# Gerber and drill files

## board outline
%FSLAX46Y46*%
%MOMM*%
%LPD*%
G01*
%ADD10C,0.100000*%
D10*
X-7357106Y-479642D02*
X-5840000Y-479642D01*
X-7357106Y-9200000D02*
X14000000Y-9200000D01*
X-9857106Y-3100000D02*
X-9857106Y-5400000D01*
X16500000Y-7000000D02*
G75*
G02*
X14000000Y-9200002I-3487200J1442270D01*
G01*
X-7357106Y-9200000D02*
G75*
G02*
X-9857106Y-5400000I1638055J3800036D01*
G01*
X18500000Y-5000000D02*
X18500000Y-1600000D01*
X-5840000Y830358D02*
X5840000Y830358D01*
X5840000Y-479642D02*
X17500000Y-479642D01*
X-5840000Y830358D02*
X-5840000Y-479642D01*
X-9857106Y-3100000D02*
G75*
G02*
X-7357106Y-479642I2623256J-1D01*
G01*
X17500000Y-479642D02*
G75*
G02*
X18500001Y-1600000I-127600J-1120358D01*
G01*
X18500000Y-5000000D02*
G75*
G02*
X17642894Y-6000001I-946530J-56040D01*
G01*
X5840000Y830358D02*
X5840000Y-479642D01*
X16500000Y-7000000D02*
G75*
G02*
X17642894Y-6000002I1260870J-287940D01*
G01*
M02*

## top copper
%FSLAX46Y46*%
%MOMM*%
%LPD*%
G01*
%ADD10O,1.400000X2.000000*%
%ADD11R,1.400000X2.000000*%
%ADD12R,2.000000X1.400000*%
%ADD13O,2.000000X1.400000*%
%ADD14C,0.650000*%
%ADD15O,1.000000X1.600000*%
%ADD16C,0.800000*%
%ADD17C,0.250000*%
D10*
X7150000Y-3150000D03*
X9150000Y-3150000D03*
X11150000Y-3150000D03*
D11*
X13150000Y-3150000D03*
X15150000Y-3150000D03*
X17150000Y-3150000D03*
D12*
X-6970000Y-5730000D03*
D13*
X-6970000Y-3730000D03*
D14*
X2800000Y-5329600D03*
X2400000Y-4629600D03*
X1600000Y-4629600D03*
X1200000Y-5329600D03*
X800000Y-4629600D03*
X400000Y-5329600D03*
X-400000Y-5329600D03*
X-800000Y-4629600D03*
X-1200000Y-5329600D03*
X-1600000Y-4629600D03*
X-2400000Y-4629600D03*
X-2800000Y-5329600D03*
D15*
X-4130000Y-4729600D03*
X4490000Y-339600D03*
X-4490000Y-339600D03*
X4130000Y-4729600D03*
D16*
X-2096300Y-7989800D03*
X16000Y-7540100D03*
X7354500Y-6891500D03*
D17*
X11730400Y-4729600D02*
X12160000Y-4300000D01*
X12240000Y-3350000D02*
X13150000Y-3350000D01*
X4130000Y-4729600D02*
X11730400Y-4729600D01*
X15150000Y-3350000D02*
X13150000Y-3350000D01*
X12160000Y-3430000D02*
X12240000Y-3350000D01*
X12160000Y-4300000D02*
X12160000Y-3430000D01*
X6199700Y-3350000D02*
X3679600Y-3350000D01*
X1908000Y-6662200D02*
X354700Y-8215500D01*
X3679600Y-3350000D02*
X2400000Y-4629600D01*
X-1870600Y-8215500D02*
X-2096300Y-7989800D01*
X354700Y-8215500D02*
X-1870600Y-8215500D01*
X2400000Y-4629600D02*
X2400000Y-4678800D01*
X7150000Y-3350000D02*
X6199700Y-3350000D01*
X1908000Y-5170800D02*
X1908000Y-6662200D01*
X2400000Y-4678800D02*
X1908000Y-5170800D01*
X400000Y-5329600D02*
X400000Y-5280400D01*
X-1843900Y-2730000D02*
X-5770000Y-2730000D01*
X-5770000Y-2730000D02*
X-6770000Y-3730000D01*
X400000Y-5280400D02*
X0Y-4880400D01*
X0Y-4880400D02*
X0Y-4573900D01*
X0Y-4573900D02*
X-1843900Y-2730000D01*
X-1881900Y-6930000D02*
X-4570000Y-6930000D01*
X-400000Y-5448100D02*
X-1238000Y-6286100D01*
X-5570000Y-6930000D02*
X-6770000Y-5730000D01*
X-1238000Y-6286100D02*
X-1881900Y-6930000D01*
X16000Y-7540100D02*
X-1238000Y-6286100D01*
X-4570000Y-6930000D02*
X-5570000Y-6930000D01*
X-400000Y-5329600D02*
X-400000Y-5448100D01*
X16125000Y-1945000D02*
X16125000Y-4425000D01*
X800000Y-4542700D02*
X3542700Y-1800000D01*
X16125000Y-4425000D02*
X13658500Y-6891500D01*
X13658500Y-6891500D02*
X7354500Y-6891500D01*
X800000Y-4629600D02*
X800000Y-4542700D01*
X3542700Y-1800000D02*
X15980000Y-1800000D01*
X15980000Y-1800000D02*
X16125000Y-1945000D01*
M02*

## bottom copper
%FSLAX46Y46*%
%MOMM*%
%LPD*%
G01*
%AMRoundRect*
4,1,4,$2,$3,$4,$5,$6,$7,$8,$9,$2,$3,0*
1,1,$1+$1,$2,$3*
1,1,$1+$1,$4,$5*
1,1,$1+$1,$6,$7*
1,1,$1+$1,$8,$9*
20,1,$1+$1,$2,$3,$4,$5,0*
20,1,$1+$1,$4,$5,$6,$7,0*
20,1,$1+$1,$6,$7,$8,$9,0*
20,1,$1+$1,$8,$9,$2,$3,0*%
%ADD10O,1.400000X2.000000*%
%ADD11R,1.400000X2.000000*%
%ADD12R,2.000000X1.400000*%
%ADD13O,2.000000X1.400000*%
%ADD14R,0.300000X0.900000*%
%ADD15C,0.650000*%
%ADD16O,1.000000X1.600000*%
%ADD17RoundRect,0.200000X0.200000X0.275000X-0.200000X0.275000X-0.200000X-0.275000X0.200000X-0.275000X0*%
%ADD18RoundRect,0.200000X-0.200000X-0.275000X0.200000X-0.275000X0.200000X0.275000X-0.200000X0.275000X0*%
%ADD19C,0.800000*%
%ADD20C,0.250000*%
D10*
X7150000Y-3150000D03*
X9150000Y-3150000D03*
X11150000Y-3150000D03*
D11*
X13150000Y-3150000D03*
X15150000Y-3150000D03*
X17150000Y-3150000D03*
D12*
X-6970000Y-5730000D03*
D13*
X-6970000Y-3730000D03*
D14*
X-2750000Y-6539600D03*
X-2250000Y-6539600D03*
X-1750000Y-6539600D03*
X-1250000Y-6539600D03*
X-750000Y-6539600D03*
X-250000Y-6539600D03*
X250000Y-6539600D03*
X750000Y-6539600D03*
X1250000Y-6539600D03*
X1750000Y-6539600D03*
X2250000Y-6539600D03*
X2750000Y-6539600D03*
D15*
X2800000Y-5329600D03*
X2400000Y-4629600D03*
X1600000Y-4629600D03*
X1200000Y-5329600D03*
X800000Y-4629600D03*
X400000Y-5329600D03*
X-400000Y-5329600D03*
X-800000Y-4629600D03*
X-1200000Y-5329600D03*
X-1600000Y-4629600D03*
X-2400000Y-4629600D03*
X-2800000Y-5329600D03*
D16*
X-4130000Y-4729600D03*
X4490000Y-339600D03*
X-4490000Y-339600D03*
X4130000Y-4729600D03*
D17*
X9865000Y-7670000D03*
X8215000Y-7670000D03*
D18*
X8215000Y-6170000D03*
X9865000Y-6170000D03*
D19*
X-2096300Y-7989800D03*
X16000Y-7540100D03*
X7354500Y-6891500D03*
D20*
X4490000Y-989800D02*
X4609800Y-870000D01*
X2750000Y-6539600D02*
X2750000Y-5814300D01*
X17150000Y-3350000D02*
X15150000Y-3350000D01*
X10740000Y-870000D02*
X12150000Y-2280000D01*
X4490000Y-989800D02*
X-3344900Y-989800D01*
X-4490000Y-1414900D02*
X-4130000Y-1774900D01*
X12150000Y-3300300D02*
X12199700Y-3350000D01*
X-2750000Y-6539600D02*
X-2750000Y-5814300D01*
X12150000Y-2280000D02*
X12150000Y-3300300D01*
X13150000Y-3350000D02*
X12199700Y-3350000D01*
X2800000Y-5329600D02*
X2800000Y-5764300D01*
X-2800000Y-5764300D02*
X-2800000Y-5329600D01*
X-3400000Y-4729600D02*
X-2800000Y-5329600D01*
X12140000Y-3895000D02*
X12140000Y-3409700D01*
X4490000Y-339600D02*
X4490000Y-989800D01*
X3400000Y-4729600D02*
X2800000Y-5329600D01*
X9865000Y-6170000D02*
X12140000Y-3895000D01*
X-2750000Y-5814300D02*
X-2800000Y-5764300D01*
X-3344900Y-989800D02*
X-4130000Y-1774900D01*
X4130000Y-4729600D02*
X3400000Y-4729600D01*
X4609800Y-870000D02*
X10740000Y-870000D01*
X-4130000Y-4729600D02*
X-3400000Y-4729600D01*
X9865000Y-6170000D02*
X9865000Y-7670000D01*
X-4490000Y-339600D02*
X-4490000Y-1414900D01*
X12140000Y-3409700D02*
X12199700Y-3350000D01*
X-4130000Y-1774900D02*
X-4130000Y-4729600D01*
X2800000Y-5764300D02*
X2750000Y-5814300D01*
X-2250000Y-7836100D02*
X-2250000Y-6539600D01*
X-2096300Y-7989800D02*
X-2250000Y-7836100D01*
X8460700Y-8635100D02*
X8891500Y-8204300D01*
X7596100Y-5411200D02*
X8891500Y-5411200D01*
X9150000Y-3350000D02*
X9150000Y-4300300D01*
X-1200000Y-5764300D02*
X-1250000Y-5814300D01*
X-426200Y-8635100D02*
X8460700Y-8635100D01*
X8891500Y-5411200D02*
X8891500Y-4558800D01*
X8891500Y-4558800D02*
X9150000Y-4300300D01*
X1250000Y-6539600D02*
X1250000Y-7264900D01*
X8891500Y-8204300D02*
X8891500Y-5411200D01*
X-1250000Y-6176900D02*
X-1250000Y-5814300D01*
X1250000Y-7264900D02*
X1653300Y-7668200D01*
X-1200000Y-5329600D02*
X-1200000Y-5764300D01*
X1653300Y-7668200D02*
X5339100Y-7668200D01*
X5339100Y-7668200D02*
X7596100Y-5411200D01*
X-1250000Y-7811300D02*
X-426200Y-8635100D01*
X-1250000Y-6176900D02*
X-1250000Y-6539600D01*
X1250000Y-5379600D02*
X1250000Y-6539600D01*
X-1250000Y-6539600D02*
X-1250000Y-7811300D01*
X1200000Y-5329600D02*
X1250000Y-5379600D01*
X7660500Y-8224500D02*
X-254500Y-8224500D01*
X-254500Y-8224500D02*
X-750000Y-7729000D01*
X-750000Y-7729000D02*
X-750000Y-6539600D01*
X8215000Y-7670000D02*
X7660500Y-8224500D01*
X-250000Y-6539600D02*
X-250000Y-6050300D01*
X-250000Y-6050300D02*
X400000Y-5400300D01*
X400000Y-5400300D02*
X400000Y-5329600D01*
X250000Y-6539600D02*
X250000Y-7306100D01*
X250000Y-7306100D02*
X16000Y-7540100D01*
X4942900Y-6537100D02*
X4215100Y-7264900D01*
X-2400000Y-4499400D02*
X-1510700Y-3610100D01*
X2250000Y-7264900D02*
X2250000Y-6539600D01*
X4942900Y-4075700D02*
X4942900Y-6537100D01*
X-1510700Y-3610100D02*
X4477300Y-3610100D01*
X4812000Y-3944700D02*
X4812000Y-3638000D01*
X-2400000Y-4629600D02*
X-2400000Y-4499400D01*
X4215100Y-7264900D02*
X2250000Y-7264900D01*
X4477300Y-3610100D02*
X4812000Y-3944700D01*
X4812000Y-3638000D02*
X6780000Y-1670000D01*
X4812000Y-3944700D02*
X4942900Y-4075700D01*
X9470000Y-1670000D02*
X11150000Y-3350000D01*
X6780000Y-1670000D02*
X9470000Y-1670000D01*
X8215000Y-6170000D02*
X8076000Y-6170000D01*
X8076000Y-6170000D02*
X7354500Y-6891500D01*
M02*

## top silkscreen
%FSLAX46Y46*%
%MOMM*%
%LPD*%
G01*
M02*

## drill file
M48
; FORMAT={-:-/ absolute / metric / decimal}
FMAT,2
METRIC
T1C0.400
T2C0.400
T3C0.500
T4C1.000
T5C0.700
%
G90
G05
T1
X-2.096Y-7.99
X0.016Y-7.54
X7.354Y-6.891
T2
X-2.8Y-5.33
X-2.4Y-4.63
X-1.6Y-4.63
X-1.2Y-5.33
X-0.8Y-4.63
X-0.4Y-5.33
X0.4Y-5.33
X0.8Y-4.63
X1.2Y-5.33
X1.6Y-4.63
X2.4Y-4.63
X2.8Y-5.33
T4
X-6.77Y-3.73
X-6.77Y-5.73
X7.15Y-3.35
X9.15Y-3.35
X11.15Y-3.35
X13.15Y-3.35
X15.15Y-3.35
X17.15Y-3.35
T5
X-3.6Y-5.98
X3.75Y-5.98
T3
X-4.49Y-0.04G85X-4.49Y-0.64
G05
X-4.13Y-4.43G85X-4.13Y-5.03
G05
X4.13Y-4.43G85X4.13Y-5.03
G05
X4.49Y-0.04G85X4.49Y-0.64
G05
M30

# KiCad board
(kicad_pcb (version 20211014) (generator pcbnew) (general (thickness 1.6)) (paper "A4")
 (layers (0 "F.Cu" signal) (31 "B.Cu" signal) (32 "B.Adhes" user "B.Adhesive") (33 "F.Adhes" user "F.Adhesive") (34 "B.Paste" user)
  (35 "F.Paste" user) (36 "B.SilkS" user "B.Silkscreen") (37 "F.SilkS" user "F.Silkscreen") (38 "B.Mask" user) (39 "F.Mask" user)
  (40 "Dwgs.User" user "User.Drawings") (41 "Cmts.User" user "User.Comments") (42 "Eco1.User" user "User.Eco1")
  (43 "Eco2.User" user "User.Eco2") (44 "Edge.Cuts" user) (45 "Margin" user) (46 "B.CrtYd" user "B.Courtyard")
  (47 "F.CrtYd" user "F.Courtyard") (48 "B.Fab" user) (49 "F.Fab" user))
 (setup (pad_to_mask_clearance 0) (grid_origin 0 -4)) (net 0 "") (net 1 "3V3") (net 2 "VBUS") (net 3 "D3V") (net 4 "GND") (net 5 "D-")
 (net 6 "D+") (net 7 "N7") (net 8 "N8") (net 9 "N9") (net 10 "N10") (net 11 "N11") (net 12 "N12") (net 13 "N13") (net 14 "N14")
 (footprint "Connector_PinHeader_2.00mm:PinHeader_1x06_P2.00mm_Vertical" (layer "F.Cu") (at 7.15 3.35 90)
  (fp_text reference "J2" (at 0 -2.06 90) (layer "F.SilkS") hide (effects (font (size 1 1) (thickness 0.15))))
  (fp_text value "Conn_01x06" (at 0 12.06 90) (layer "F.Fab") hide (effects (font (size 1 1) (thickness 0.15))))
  (pad "1" thru_hole oval locked (at 0 0 90) (size 2 1.4) (drill 1 (offset 0.2 0)) (layers *.Cu *.Mask) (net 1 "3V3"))
  (pad "2" thru_hole oval locked (at 0 2 90) (size 2 1.4) (drill 1 (offset 0.2 0)) (layers *.Cu *.Mask) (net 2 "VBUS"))
  (pad "3" thru_hole oval locked (at 0 4 90) (size 2 1.4) (drill 1 (offset 0.2 0)) (layers *.Cu *.Mask) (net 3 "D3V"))
  (pad "4" thru_hole rect locked (at 0 6 90) (size 2 1.4) (drill 1 (offset 0.2 0)) (layers *.Cu *.Mask) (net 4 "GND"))
  (pad "5" thru_hole rect locked (at 0 8 90) (size 2 1.4) (drill 1 (offset 0.2 0)) (layers *.Cu *.Mask) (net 4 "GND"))
  (pad "6" thru_hole rect locked (at 0 10 90) (size 2 1.4) (drill 1 (offset 0.2 0)) (layers *.Cu *.Mask) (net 4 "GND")))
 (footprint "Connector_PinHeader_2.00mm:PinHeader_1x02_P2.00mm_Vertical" (layer "F.Cu") (at -6.77 5.73 180)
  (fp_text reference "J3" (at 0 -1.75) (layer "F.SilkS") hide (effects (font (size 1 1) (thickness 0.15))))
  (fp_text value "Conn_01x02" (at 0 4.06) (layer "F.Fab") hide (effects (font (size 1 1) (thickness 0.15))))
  (pad "1" thru_hole rect locked (at 0 0 180) (size 2 1.4) (drill 1 (offset 0.2 0)) (layers *.Cu *.Mask) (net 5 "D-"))
  (pad "2" thru_hole oval locked (at 0 2 180) (size 2 1.4) (drill 1 (offset 0.2 0)) (layers *.Cu *.Mask) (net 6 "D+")))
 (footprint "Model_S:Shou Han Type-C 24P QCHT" (layer "B.Cu") (at 0 -1.5204)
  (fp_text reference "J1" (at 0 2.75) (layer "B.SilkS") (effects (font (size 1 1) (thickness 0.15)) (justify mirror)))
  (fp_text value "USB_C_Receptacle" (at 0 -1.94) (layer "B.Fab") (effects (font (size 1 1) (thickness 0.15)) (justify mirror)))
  (pad "" np_thru_hole circle (at -3.6 7.5) (size 0.7 0.7) (drill 0.7) (layers *.Cu *.Mask))
  (pad "" np_thru_hole circle (at 3.75 7.5) (size 0.7 0.7) (drill 0.7) (layers *.Cu *.Mask))
  (pad "A1" smd rect (at -2.75 8.06) (size 0.3 0.9) (layers "B.Cu" "B.Paste" "B.Mask") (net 4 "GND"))
  (pad "A2" smd rect (at -2.25 8.06) (size 0.3 0.9) (layers "B.Cu" "B.Paste" "B.Mask") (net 1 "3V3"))
  (pad "A3" smd rect (at -1.75 8.06) (size 0.3 0.9) (layers "B.Cu" "B.Paste" "B.Mask") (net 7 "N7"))
  (pad "A4" smd rect (at -1.25 8.06) (size 0.3 0.9) (layers "B.Cu" "B.Paste" "B.Mask") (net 2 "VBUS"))
  (pad "A5" smd rect (at -0.75 8.06) (size 0.3 0.9) (layers "B.Cu" "B.Paste" "B.Mask") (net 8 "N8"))
  (pad "A6" smd rect (at -0.25 8.06) (size 0.3 0.9) (layers "B.Cu" "B.Paste" "B.Mask") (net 6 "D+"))
  (pad "A7" smd rect (at 0.25 8.06) (size 0.3 0.9) (layers "B.Cu" "B.Paste" "B.Mask") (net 5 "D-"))
  (pad "A8" smd rect (at 0.75 8.06) (size 0.3 0.9) (layers "B.Cu" "B.Paste" "B.Mask") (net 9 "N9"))
  (pad "A9" smd rect (at 1.25 8.06) (size 0.3 0.9) (layers "B.Cu" "B.Paste" "B.Mask") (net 2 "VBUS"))
  (pad "A10" smd rect (at 1.75 8.06) (size 0.3 0.9) (layers "B.Cu" "B.Paste" "B.Mask") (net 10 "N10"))
  (pad "A11" smd rect (at 2.25 8.06) (size 0.3 0.9) (layers "B.Cu" "B.Paste" "B.Mask") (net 3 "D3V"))
  (pad "A12" smd rect (at 2.75 8.06) (size 0.3 0.9) (layers "B.Cu" "B.Paste" "B.Mask") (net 4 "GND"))
  (pad "B1" thru_hole circle (at 2.8 6.85) (size 0.65 0.65) (drill 0.4) (layers *.Cu *.Mask) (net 4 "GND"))
  (pad "B2" thru_hole circle (at 2.4 6.15) (size 0.65 0.65) (drill 0.4) (layers *.Cu *.Mask) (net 1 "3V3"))
  (pad "B3" thru_hole circle (at 1.6 6.15) (size 0.65 0.65) (drill 0.4) (layers *.Cu *.Mask) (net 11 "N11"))
  (pad "B4" thru_hole circle (at 1.2 6.85) (size 0.65 0.65) (drill 0.4) (layers *.Cu *.Mask) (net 2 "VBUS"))
  (pad "B5" thru_hole circle (at 0.8 6.15) (size 0.65 0.65) (drill 0.4) (layers *.Cu *.Mask) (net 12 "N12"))
  (pad "B6" thru_hole circle (at 0.4 6.85) (size 0.65 0.65) (drill 0.4) (layers *.Cu *.Mask) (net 6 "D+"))
  (pad "B7" thru_hole circle (at -0.4 6.85) (size 0.65 0.65) (drill 0.4) (layers *.Cu *.Mask) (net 5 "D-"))
  (pad "B8" thru_hole circle (at -0.8 6.15) (size 0.65 0.65) (drill 0.4) (layers *.Cu *.Mask) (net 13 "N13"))
  (pad "B9" thru_hole circle (at -1.2 6.85) (size 0.65 0.65) (drill 0.4) (layers *.Cu *.Mask) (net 2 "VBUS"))
  (pad "B10" thru_hole circle (at -1.6 6.15) (size 0.65 0.65) (drill 0.4) (layers *.Cu *.Mask) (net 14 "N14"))
  (pad "B11" thru_hole circle (at -2.4 6.15) (size 0.65 0.65) (drill 0.4) (layers *.Cu *.Mask) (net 3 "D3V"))
  (pad "B12" thru_hole circle (at -2.8 6.85) (size 0.65 0.65) (drill 0.4) (layers *.Cu *.Mask) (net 4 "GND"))
  (pad "S1" thru_hole oval (at -4.13 6.25) (size 1 1.6) (drill oval 0.5 1.1) (layers *.Cu *.Mask) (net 4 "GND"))
  (pad "S1" thru_hole oval (at 4.49 1.86) (size 1 1.6) (drill oval 0.5 1.1) (layers *.Cu *.Mask) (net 4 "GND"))
  (pad "S1" thru_hole oval (at -4.49 1.86) (size 1 1.6) (drill oval 0.5 1.1) (layers *.Cu *.Mask) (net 4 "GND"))
  (pad "S1" thru_hole oval (at 4.13 6.25) (size 1 1.6) (drill oval 0.5 1.1) (layers *.Cu *.Mask) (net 4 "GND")))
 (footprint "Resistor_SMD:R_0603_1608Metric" (layer "B.Cu") (at 9.04 7.67 180)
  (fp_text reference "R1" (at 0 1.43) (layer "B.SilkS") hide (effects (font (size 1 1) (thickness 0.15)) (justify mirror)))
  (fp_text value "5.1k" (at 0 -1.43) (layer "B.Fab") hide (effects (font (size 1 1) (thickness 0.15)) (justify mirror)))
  (pad "1" smd roundrect locked (at -0.825 0 180) (size 0.8 0.95) (layers "B.Cu" "B.Paste" "B.Mask") (roundrect_rratio 0.25) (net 4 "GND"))
  (pad "2" smd roundrect locked (at 0.825 0 180) (size 0.8 0.95) (layers "B.Cu" "B.Paste" "B.Mask") (roundrect_rratio 0.25) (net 8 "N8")))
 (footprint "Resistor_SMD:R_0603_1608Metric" (layer "B.Cu") (at 9.04 6.17)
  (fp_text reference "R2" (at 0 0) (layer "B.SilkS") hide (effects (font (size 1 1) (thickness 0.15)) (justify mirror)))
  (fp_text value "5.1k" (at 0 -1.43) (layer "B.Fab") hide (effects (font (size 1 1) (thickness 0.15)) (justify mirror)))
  (pad "1" smd roundrect locked (at -0.825 0) (size 0.8 0.95) (layers "B.Cu" "B.Paste" "B.Mask") (roundrect_rratio 0.25) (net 12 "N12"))
  (pad "2" smd roundrect locked (at 0.825 0) (size 0.8 0.95) (layers "B.Cu" "B.Paste" "B.Mask") (roundrect_rratio 0.25) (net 4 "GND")))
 (gr_line (start -7.357106 0.479642) (end -5.84 0.479642) (layer "Edge.Cuts") (width 0.1))
 (gr_line (start -7.357106 9.2) (end 14 9.2) (layer "Edge.Cuts") (width 0.1))
 (gr_line (start -9.857106 3.1) (end -9.857106 5.4) (layer "Edge.Cuts") (width 0.1))
 (gr_arc (start 16.5 7) (mid 15.505803 8.390686) (end 14 9.2) (layer "Edge.Cuts") (width 0.1))
 (gr_arc (start -7.357106 9.2) (mid -9.176053 7.674307) (end -9.857106 5.4) (layer "Edge.Cuts") (width 0.1))
 (gr_line (start 18.5 5) (end 18.5 1.6) (layer "Edge.Cuts") (width 0.1))
 (gr_line (start -5.84 -0.830358) (end 5.84 -0.830358) (layer "Edge.Cuts") (width 0.1))
 (gr_line (start 5.84 0.479642) (end 17.5 0.479642) (layer "Edge.Cuts") (width 0.1))
 (gr_line (start -5.84 -0.830358) (end -5.84 0.479642) (layer "Edge.Cuts") (width 0.1))
 (gr_arc (start -9.857106 3.1) (mid -9.131849 1.28918) (end -7.357106 0.479642) (layer "Edge.Cuts") (width 0.1))
 (gr_arc (start 17.5 0.479642) (mid 18.213632 0.849137) (end 18.5 1.6) (layer "Edge.Cuts") (width 0.1))
 (gr_arc (start 18.5 5) (mid 18.273401 5.673097) (end 17.642894 6) (layer "Edge.Cuts") (width 0.1))
 (gr_line (start 5.84 -0.830358) (end 5.84 0.479642) (layer "Edge.Cuts") (width 0.1))
 (gr_arc (start 16.5 7) (mid 16.909223 6.314595) (end 17.642894 6) (layer "Edge.Cuts") (width 0.1))
 (segment (start 11.7304 4.7296) (end 12.16 4.3) (width 0.25) (layer "F.Cu") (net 4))
 (segment (start 12.24 3.35) (end 13.15 3.35) (width 0.25) (layer "F.Cu") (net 4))
 (segment (start 4.13 4.7296) (end 11.7304 4.7296) (width 0.25) (layer "F.Cu") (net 4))
 (segment (start 15.15 3.35) (end 13.15 3.35) (width 0.25) (layer "F.Cu") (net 4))
 (segment (start 12.16 3.43) (end 12.24 3.35) (width 0.25) (layer "F.Cu") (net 4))
 (segment (start 12.16 4.3) (end 12.16 3.43) (width 0.25) (layer "F.Cu") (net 4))
 (segment (start 4.49 0.9898) (end 4.6098 0.87) (width 0.25) (layer "B.Cu") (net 4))
 (segment (start 2.75 6.5396) (end 2.75 5.8143) (width 0.25) (layer "B.Cu") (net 4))
 (segment (start 17.15 3.35) (end 15.15 3.35) (width 0.25) (layer "B.Cu") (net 4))
 (segment (start 10.74 0.87) (end 12.15 2.28) (width 0.25) (layer "B.Cu") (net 4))
 (segment (start 4.49 0.9898) (end -3.3449 0.9898) (width 0.25) (layer "B.Cu") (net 4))
 (segment (start -4.49 1.4149) (end -4.13 1.7749) (width 0.25) (layer "B.Cu") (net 4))
 (segment (start 12.15 3.3003) (end 12.1997 3.35) (width 0.25) (layer "B.Cu") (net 4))
 (segment (start -2.75 6.5396) (end -2.75 5.8143) (width 0.25) (layer "B.Cu") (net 4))
 (segment (start 12.15 2.28) (end 12.15 3.3003) (width 0.25) (layer "B.Cu") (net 4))
 (segment (start 13.15 3.35) (end 12.1997 3.35) (width 0.25) (layer "B.Cu") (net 4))
 (segment (start 2.8 5.3296) (end 2.8 5.7643) (width 0.25) (layer "B.Cu") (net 4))
 (segment (start -2.8 5.7643) (end -2.8 5.3296) (width 0.25) (layer "B.Cu") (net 4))
 (segment (start -3.4 4.7296) (end -2.8 5.3296) (width 0.25) (layer "B.Cu") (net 4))
 (segment (start 12.14 3.895) (end 12.14 3.4097) (width 0.25) (layer "B.Cu") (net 4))
 (segment (start 4.49 0.3396) (end 4.49 0.9898) (width 0.25) (layer "B.Cu") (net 4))
 (segment (start 3.4 4.7296) (end 2.8 5.3296) (width 0.25) (layer "B.Cu") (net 4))
 (segment (start 9.865 6.17) (end 12.14 3.895) (width 0.25) (layer "B.Cu") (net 4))
 (segment (start -2.75 5.8143) (end -2.8 5.7643) (width 0.25) (layer "B.Cu") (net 4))
 (segment (start -3.3449 0.9898) (end -4.13 1.7749) (width 0.25) (layer "B.Cu") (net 4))
 (segment (start 4.13 4.7296) (end 3.4 4.7296) (width 0.25) (layer "B.Cu") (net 4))
 (segment (start 4.6098 0.87) (end 10.74 0.87) (width 0.25) (layer "B.Cu") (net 4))
 (segment (start -4.13 4.7296) (end -3.4 4.7296) (width 0.25) (layer "B.Cu") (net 4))
 (segment (start 9.865 6.17) (end 9.865 7.67) (width 0.25) (layer "B.Cu") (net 4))
 (segment (start -4.49 0.3396) (end -4.49 1.4149) (width 0.25) (layer "B.Cu") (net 4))
 (segment (start 12.14 3.4097) (end 12.1997 3.35) (width 0.25) (layer "B.Cu") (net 4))
 (segment (start -4.13 1.7749) (end -4.13 4.7296) (width 0.25) (layer "B.Cu") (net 4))
 (segment (start 2.8 5.7643) (end 2.75 5.8143) (width 0.25) (layer "B.Cu") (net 4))
 (segment (start 6.1997 3.35) (end 3.6796 3.35) (width 0.25) (layer "F.Cu") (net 1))
 (segment (start 1.908 6.6622) (end 0.3547 8.2155) (width 0.25) (layer "F.Cu") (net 1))
 (segment (start 3.6796 3.35) (end 2.4 4.6296) (width 0.25) (layer "F.Cu") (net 1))
 (segment (start -1.8706 8.2155) (end -2.0963 7.9898) (width 0.25) (layer "F.Cu") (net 1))
 (segment (start 0.3547 8.2155) (end -1.8706 8.2155) (width 0.25) (layer "F.Cu") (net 1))
 (segment (start 2.4 4.6296) (end 2.4 4.6788) (width 0.25) (layer "F.Cu") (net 1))
 (segment (start 7.15 3.35) (end 6.1997 3.35) (width 0.25) (layer "F.Cu") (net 1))
 (segment (start 1.908 5.1708) (end 1.908 6.6622) (width 0.25) (layer "F.Cu") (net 1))
 (segment (start 2.4 4.6788) (end 1.908 5.1708) (width 0.25) (layer "F.Cu") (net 1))
 (via (at -2.0963 7.9898) (size 0.8) (drill 0.4) (layers "F.Cu" "B.Cu") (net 1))
 (segment (start -2.25 7.8361) (end -2.25 6.5396) (width 0.25) (layer "B.Cu") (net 1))
 (segment (start -2.0963 7.9898) (end -2.25 7.8361) (width 0.25) (layer "B.Cu") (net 1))
 (segment (start 8.4607 8.6351) (end 8.8915 8.2043) (width 0.25) (layer "B.Cu") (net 2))
 (segment (start 7.5961 5.4112) (end 8.8915 5.4112) (width 0.25) (layer "B.Cu") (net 2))
 (segment (start 9.15 3.35) (end 9.15 4.3003) (width 0.25) (layer "B.Cu") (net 2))
 (segment (start -1.2 5.7643) (end -1.25 5.8143) (width 0.25) (layer "B.Cu") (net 2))
 (segment (start -0.4262 8.6351) (end 8.4607 8.6351) (width 0.25) (layer "B.Cu") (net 2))
 (segment (start 8.8915 5.4112) (end 8.8915 4.5588) (width 0.25) (layer "B.Cu") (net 2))
 (segment (start 8.8915 4.5588) (end 9.15 4.3003) (width 0.25) (layer "B.Cu") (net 2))
 (segment (start 1.25 6.5396) (end 1.25 7.2649) (width 0.25) (layer "B.Cu") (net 2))
 (segment (start 8.8915 8.2043) (end 8.8915 5.4112) (width 0.25) (layer "B.Cu") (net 2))
 (segment (start -1.25 6.1769) (end -1.25 5.8143) (width 0.25) (layer "B.Cu") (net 2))
 (segment (start 1.25 7.2649) (end 1.6533 7.6682) (width 0.25) (layer "B.Cu") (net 2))
 (segment (start -1.2 5.3296) (end -1.2 5.7643) (width 0.25) (layer "B.Cu") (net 2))
 (segment (start 1.6533 7.6682) (end 5.3391 7.6682) (width 0.25) (layer "B.Cu") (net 2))
 (segment (start 5.3391 7.6682) (end 7.5961 5.4112) (width 0.25) (layer "B.Cu") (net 2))
 (segment (start -1.25 7.8113) (end -0.4262 8.6351) (width 0.25) (layer "B.Cu") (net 2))
 (segment (start -1.25 6.1769) (end -1.25 6.5396) (width 0.25) (layer "B.Cu") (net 2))
 (segment (start 1.25 5.3796) (end 1.25 6.5396) (width 0.25) (layer "B.Cu") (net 2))
 (segment (start -1.25 6.5396) (end -1.25 7.8113) (width 0.25) (layer "B.Cu") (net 2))
 (segment (start 1.2 5.3296) (end 1.25 5.3796) (width 0.25) (layer "B.Cu") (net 2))
 (segment (start 7.6605 8.2245) (end -0.2545 8.2245) (width 0.25) (layer "B.Cu") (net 8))
 (segment (start -0.2545 8.2245) (end -0.75 7.729) (width 0.25) (layer "B.Cu") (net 8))
 (segment (start -0.75 7.729) (end -0.75 6.5396) (width 0.25) (layer "B.Cu") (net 8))
 (segment (start 8.215 7.67) (end 7.6605 8.2245) (width 0.25) (layer "B.Cu") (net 8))
 (segment (start 0.4 5.3296) (end 0.4 5.2804) (width 0.25) (layer "F.Cu") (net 6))
 (segment (start -1.8439 2.73) (end -5.77 2.73) (width 0.25) (layer "F.Cu") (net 6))
 (segment (start -5.77 2.73) (end -6.77 3.73) (width 0.25) (layer "F.Cu") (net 6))
 (segment (start 0.4 5.2804) (end 0 4.8804) (width 0.25) (layer "F.Cu") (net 6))
 (segment (start 0 4.8804) (end 0 4.5739) (width 0.25) (layer "F.Cu") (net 6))
 (segment (start 0 4.5739) (end -1.8439 2.73) (width 0.25) (layer "F.Cu") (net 6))
 (segment (start -0.25 6.5396) (end -0.25 6.0503) (width 0.25) (layer "B.Cu") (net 6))
 (segment (start -0.25 6.0503) (end 0.4 5.4003) (width 0.25) (layer "B.Cu") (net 6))
 (segment (start 0.4 5.4003) (end 0.4 5.3296) (width 0.25) (layer "B.Cu") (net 6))
 (segment (start -1.8819 6.93) (end -4.57 6.93) (width 0.25) (layer "F.Cu") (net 5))
 (segment (start -0.4 5.4481) (end -1.238 6.2861) (width 0.25) (layer "F.Cu") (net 5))
 (segment (start -5.57 6.93) (end -6.77 5.73) (width 0.25) (layer "F.Cu") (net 5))
 (segment (start -1.238 6.2861) (end -1.8819 6.93) (width 0.25) (layer "F.Cu") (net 5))
 (segment (start 0.016 7.5401) (end -1.238 6.2861) (width 0.25) (layer "F.Cu") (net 5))
 (segment (start -4.57 6.93) (end -5.57 6.93) (width 0.25) (layer "F.Cu") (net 5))
 (segment (start -0.4 5.3296) (end -0.4 5.4481) (width 0.25) (layer "F.Cu") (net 5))
 (via (at 0.016 7.5401) (size 0.8) (drill 0.4) (layers "F.Cu" "B.Cu") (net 5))
 (segment (start 0.25 6.5396) (end 0.25 7.3061) (width 0.25) (layer "B.Cu") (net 5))
 (segment (start 0.25 7.3061) (end 0.016 7.5401) (width 0.25) (layer "B.Cu") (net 5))
 (segment (start 4.9429 6.5371) (end 4.2151 7.2649) (width 0.25) (layer "B.Cu") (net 3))
 (segment (start -2.4 4.4994) (end -1.5107 3.6101) (width 0.25) (layer "B.Cu") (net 3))
 (segment (start 2.25 7.2649) (end 2.25 6.5396) (width 0.25) (layer "B.Cu") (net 3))
 (segment (start 4.9429 4.0757) (end 4.9429 6.5371) (width 0.25) (layer "B.Cu") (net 3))
 (segment (start -1.5107 3.6101) (end 4.4773 3.6101) (width 0.25) (layer "B.Cu") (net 3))
 (segment (start 4.812 3.9447) (end 4.812 3.638) (width 0.25) (layer "B.Cu") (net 3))
 (segment (start -2.4 4.6296) (end -2.4 4.4994) (width 0.25) (layer "B.Cu") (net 3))
 (segment (start 4.2151 7.2649) (end 2.25 7.2649) (width 0.25) (layer "B.Cu") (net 3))
 (segment (start 4.4773 3.6101) (end 4.812 3.9447) (width 0.25) (layer "B.Cu") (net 3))
 (segment (start 4.812 3.638) (end 6.78 1.67) (width 0.25) (layer "B.Cu") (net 3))
 (segment (start 4.812 3.9447) (end 4.9429 4.0757) (width 0.25) (layer "B.Cu") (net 3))
 (segment (start 9.47 1.67) (end 11.15 3.35) (width 0.25) (layer "B.Cu") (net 3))
 (segment (start 6.78 1.67) (end 9.47 1.67) (width 0.25) (layer "B.Cu") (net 3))
 (segment (start 16.125 1.945) (end 16.125 4.425) (width 0.25) (layer "F.Cu") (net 12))
 (segment (start 0.8 4.5427) (end 3.5427 1.8) (width 0.25) (layer "F.Cu") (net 12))
 (segment (start 16.125 4.425) (end 13.6585 6.8915) (width 0.25) (layer "F.Cu") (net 12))
 (segment (start 13.6585 6.8915) (end 7.3545 6.8915) (width 0.25) (layer "F.Cu") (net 12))
 (segment (start 0.8 4.6296) (end 0.8 4.5427) (width 0.25) (layer "F.Cu") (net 12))
 (segment (start 3.5427 1.8) (end 15.98 1.8) (width 0.25) (layer "F.Cu") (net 12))
 (segment (start 15.98 1.8) (end 16.125 1.945) (width 0.25) (layer "F.Cu") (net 12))
 (via (at 7.3545 6.8915) (size 0.8) (drill 0.4) (layers "F.Cu" "B.Cu") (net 12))
 (segment (start 8.215 6.17) (end 8.076 6.17) (width 0.25) (layer "B.Cu") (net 12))
 (segment (start 8.076 6.17) (end 7.3545 6.8915) (width 0.25) (layer "B.Cu") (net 12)))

